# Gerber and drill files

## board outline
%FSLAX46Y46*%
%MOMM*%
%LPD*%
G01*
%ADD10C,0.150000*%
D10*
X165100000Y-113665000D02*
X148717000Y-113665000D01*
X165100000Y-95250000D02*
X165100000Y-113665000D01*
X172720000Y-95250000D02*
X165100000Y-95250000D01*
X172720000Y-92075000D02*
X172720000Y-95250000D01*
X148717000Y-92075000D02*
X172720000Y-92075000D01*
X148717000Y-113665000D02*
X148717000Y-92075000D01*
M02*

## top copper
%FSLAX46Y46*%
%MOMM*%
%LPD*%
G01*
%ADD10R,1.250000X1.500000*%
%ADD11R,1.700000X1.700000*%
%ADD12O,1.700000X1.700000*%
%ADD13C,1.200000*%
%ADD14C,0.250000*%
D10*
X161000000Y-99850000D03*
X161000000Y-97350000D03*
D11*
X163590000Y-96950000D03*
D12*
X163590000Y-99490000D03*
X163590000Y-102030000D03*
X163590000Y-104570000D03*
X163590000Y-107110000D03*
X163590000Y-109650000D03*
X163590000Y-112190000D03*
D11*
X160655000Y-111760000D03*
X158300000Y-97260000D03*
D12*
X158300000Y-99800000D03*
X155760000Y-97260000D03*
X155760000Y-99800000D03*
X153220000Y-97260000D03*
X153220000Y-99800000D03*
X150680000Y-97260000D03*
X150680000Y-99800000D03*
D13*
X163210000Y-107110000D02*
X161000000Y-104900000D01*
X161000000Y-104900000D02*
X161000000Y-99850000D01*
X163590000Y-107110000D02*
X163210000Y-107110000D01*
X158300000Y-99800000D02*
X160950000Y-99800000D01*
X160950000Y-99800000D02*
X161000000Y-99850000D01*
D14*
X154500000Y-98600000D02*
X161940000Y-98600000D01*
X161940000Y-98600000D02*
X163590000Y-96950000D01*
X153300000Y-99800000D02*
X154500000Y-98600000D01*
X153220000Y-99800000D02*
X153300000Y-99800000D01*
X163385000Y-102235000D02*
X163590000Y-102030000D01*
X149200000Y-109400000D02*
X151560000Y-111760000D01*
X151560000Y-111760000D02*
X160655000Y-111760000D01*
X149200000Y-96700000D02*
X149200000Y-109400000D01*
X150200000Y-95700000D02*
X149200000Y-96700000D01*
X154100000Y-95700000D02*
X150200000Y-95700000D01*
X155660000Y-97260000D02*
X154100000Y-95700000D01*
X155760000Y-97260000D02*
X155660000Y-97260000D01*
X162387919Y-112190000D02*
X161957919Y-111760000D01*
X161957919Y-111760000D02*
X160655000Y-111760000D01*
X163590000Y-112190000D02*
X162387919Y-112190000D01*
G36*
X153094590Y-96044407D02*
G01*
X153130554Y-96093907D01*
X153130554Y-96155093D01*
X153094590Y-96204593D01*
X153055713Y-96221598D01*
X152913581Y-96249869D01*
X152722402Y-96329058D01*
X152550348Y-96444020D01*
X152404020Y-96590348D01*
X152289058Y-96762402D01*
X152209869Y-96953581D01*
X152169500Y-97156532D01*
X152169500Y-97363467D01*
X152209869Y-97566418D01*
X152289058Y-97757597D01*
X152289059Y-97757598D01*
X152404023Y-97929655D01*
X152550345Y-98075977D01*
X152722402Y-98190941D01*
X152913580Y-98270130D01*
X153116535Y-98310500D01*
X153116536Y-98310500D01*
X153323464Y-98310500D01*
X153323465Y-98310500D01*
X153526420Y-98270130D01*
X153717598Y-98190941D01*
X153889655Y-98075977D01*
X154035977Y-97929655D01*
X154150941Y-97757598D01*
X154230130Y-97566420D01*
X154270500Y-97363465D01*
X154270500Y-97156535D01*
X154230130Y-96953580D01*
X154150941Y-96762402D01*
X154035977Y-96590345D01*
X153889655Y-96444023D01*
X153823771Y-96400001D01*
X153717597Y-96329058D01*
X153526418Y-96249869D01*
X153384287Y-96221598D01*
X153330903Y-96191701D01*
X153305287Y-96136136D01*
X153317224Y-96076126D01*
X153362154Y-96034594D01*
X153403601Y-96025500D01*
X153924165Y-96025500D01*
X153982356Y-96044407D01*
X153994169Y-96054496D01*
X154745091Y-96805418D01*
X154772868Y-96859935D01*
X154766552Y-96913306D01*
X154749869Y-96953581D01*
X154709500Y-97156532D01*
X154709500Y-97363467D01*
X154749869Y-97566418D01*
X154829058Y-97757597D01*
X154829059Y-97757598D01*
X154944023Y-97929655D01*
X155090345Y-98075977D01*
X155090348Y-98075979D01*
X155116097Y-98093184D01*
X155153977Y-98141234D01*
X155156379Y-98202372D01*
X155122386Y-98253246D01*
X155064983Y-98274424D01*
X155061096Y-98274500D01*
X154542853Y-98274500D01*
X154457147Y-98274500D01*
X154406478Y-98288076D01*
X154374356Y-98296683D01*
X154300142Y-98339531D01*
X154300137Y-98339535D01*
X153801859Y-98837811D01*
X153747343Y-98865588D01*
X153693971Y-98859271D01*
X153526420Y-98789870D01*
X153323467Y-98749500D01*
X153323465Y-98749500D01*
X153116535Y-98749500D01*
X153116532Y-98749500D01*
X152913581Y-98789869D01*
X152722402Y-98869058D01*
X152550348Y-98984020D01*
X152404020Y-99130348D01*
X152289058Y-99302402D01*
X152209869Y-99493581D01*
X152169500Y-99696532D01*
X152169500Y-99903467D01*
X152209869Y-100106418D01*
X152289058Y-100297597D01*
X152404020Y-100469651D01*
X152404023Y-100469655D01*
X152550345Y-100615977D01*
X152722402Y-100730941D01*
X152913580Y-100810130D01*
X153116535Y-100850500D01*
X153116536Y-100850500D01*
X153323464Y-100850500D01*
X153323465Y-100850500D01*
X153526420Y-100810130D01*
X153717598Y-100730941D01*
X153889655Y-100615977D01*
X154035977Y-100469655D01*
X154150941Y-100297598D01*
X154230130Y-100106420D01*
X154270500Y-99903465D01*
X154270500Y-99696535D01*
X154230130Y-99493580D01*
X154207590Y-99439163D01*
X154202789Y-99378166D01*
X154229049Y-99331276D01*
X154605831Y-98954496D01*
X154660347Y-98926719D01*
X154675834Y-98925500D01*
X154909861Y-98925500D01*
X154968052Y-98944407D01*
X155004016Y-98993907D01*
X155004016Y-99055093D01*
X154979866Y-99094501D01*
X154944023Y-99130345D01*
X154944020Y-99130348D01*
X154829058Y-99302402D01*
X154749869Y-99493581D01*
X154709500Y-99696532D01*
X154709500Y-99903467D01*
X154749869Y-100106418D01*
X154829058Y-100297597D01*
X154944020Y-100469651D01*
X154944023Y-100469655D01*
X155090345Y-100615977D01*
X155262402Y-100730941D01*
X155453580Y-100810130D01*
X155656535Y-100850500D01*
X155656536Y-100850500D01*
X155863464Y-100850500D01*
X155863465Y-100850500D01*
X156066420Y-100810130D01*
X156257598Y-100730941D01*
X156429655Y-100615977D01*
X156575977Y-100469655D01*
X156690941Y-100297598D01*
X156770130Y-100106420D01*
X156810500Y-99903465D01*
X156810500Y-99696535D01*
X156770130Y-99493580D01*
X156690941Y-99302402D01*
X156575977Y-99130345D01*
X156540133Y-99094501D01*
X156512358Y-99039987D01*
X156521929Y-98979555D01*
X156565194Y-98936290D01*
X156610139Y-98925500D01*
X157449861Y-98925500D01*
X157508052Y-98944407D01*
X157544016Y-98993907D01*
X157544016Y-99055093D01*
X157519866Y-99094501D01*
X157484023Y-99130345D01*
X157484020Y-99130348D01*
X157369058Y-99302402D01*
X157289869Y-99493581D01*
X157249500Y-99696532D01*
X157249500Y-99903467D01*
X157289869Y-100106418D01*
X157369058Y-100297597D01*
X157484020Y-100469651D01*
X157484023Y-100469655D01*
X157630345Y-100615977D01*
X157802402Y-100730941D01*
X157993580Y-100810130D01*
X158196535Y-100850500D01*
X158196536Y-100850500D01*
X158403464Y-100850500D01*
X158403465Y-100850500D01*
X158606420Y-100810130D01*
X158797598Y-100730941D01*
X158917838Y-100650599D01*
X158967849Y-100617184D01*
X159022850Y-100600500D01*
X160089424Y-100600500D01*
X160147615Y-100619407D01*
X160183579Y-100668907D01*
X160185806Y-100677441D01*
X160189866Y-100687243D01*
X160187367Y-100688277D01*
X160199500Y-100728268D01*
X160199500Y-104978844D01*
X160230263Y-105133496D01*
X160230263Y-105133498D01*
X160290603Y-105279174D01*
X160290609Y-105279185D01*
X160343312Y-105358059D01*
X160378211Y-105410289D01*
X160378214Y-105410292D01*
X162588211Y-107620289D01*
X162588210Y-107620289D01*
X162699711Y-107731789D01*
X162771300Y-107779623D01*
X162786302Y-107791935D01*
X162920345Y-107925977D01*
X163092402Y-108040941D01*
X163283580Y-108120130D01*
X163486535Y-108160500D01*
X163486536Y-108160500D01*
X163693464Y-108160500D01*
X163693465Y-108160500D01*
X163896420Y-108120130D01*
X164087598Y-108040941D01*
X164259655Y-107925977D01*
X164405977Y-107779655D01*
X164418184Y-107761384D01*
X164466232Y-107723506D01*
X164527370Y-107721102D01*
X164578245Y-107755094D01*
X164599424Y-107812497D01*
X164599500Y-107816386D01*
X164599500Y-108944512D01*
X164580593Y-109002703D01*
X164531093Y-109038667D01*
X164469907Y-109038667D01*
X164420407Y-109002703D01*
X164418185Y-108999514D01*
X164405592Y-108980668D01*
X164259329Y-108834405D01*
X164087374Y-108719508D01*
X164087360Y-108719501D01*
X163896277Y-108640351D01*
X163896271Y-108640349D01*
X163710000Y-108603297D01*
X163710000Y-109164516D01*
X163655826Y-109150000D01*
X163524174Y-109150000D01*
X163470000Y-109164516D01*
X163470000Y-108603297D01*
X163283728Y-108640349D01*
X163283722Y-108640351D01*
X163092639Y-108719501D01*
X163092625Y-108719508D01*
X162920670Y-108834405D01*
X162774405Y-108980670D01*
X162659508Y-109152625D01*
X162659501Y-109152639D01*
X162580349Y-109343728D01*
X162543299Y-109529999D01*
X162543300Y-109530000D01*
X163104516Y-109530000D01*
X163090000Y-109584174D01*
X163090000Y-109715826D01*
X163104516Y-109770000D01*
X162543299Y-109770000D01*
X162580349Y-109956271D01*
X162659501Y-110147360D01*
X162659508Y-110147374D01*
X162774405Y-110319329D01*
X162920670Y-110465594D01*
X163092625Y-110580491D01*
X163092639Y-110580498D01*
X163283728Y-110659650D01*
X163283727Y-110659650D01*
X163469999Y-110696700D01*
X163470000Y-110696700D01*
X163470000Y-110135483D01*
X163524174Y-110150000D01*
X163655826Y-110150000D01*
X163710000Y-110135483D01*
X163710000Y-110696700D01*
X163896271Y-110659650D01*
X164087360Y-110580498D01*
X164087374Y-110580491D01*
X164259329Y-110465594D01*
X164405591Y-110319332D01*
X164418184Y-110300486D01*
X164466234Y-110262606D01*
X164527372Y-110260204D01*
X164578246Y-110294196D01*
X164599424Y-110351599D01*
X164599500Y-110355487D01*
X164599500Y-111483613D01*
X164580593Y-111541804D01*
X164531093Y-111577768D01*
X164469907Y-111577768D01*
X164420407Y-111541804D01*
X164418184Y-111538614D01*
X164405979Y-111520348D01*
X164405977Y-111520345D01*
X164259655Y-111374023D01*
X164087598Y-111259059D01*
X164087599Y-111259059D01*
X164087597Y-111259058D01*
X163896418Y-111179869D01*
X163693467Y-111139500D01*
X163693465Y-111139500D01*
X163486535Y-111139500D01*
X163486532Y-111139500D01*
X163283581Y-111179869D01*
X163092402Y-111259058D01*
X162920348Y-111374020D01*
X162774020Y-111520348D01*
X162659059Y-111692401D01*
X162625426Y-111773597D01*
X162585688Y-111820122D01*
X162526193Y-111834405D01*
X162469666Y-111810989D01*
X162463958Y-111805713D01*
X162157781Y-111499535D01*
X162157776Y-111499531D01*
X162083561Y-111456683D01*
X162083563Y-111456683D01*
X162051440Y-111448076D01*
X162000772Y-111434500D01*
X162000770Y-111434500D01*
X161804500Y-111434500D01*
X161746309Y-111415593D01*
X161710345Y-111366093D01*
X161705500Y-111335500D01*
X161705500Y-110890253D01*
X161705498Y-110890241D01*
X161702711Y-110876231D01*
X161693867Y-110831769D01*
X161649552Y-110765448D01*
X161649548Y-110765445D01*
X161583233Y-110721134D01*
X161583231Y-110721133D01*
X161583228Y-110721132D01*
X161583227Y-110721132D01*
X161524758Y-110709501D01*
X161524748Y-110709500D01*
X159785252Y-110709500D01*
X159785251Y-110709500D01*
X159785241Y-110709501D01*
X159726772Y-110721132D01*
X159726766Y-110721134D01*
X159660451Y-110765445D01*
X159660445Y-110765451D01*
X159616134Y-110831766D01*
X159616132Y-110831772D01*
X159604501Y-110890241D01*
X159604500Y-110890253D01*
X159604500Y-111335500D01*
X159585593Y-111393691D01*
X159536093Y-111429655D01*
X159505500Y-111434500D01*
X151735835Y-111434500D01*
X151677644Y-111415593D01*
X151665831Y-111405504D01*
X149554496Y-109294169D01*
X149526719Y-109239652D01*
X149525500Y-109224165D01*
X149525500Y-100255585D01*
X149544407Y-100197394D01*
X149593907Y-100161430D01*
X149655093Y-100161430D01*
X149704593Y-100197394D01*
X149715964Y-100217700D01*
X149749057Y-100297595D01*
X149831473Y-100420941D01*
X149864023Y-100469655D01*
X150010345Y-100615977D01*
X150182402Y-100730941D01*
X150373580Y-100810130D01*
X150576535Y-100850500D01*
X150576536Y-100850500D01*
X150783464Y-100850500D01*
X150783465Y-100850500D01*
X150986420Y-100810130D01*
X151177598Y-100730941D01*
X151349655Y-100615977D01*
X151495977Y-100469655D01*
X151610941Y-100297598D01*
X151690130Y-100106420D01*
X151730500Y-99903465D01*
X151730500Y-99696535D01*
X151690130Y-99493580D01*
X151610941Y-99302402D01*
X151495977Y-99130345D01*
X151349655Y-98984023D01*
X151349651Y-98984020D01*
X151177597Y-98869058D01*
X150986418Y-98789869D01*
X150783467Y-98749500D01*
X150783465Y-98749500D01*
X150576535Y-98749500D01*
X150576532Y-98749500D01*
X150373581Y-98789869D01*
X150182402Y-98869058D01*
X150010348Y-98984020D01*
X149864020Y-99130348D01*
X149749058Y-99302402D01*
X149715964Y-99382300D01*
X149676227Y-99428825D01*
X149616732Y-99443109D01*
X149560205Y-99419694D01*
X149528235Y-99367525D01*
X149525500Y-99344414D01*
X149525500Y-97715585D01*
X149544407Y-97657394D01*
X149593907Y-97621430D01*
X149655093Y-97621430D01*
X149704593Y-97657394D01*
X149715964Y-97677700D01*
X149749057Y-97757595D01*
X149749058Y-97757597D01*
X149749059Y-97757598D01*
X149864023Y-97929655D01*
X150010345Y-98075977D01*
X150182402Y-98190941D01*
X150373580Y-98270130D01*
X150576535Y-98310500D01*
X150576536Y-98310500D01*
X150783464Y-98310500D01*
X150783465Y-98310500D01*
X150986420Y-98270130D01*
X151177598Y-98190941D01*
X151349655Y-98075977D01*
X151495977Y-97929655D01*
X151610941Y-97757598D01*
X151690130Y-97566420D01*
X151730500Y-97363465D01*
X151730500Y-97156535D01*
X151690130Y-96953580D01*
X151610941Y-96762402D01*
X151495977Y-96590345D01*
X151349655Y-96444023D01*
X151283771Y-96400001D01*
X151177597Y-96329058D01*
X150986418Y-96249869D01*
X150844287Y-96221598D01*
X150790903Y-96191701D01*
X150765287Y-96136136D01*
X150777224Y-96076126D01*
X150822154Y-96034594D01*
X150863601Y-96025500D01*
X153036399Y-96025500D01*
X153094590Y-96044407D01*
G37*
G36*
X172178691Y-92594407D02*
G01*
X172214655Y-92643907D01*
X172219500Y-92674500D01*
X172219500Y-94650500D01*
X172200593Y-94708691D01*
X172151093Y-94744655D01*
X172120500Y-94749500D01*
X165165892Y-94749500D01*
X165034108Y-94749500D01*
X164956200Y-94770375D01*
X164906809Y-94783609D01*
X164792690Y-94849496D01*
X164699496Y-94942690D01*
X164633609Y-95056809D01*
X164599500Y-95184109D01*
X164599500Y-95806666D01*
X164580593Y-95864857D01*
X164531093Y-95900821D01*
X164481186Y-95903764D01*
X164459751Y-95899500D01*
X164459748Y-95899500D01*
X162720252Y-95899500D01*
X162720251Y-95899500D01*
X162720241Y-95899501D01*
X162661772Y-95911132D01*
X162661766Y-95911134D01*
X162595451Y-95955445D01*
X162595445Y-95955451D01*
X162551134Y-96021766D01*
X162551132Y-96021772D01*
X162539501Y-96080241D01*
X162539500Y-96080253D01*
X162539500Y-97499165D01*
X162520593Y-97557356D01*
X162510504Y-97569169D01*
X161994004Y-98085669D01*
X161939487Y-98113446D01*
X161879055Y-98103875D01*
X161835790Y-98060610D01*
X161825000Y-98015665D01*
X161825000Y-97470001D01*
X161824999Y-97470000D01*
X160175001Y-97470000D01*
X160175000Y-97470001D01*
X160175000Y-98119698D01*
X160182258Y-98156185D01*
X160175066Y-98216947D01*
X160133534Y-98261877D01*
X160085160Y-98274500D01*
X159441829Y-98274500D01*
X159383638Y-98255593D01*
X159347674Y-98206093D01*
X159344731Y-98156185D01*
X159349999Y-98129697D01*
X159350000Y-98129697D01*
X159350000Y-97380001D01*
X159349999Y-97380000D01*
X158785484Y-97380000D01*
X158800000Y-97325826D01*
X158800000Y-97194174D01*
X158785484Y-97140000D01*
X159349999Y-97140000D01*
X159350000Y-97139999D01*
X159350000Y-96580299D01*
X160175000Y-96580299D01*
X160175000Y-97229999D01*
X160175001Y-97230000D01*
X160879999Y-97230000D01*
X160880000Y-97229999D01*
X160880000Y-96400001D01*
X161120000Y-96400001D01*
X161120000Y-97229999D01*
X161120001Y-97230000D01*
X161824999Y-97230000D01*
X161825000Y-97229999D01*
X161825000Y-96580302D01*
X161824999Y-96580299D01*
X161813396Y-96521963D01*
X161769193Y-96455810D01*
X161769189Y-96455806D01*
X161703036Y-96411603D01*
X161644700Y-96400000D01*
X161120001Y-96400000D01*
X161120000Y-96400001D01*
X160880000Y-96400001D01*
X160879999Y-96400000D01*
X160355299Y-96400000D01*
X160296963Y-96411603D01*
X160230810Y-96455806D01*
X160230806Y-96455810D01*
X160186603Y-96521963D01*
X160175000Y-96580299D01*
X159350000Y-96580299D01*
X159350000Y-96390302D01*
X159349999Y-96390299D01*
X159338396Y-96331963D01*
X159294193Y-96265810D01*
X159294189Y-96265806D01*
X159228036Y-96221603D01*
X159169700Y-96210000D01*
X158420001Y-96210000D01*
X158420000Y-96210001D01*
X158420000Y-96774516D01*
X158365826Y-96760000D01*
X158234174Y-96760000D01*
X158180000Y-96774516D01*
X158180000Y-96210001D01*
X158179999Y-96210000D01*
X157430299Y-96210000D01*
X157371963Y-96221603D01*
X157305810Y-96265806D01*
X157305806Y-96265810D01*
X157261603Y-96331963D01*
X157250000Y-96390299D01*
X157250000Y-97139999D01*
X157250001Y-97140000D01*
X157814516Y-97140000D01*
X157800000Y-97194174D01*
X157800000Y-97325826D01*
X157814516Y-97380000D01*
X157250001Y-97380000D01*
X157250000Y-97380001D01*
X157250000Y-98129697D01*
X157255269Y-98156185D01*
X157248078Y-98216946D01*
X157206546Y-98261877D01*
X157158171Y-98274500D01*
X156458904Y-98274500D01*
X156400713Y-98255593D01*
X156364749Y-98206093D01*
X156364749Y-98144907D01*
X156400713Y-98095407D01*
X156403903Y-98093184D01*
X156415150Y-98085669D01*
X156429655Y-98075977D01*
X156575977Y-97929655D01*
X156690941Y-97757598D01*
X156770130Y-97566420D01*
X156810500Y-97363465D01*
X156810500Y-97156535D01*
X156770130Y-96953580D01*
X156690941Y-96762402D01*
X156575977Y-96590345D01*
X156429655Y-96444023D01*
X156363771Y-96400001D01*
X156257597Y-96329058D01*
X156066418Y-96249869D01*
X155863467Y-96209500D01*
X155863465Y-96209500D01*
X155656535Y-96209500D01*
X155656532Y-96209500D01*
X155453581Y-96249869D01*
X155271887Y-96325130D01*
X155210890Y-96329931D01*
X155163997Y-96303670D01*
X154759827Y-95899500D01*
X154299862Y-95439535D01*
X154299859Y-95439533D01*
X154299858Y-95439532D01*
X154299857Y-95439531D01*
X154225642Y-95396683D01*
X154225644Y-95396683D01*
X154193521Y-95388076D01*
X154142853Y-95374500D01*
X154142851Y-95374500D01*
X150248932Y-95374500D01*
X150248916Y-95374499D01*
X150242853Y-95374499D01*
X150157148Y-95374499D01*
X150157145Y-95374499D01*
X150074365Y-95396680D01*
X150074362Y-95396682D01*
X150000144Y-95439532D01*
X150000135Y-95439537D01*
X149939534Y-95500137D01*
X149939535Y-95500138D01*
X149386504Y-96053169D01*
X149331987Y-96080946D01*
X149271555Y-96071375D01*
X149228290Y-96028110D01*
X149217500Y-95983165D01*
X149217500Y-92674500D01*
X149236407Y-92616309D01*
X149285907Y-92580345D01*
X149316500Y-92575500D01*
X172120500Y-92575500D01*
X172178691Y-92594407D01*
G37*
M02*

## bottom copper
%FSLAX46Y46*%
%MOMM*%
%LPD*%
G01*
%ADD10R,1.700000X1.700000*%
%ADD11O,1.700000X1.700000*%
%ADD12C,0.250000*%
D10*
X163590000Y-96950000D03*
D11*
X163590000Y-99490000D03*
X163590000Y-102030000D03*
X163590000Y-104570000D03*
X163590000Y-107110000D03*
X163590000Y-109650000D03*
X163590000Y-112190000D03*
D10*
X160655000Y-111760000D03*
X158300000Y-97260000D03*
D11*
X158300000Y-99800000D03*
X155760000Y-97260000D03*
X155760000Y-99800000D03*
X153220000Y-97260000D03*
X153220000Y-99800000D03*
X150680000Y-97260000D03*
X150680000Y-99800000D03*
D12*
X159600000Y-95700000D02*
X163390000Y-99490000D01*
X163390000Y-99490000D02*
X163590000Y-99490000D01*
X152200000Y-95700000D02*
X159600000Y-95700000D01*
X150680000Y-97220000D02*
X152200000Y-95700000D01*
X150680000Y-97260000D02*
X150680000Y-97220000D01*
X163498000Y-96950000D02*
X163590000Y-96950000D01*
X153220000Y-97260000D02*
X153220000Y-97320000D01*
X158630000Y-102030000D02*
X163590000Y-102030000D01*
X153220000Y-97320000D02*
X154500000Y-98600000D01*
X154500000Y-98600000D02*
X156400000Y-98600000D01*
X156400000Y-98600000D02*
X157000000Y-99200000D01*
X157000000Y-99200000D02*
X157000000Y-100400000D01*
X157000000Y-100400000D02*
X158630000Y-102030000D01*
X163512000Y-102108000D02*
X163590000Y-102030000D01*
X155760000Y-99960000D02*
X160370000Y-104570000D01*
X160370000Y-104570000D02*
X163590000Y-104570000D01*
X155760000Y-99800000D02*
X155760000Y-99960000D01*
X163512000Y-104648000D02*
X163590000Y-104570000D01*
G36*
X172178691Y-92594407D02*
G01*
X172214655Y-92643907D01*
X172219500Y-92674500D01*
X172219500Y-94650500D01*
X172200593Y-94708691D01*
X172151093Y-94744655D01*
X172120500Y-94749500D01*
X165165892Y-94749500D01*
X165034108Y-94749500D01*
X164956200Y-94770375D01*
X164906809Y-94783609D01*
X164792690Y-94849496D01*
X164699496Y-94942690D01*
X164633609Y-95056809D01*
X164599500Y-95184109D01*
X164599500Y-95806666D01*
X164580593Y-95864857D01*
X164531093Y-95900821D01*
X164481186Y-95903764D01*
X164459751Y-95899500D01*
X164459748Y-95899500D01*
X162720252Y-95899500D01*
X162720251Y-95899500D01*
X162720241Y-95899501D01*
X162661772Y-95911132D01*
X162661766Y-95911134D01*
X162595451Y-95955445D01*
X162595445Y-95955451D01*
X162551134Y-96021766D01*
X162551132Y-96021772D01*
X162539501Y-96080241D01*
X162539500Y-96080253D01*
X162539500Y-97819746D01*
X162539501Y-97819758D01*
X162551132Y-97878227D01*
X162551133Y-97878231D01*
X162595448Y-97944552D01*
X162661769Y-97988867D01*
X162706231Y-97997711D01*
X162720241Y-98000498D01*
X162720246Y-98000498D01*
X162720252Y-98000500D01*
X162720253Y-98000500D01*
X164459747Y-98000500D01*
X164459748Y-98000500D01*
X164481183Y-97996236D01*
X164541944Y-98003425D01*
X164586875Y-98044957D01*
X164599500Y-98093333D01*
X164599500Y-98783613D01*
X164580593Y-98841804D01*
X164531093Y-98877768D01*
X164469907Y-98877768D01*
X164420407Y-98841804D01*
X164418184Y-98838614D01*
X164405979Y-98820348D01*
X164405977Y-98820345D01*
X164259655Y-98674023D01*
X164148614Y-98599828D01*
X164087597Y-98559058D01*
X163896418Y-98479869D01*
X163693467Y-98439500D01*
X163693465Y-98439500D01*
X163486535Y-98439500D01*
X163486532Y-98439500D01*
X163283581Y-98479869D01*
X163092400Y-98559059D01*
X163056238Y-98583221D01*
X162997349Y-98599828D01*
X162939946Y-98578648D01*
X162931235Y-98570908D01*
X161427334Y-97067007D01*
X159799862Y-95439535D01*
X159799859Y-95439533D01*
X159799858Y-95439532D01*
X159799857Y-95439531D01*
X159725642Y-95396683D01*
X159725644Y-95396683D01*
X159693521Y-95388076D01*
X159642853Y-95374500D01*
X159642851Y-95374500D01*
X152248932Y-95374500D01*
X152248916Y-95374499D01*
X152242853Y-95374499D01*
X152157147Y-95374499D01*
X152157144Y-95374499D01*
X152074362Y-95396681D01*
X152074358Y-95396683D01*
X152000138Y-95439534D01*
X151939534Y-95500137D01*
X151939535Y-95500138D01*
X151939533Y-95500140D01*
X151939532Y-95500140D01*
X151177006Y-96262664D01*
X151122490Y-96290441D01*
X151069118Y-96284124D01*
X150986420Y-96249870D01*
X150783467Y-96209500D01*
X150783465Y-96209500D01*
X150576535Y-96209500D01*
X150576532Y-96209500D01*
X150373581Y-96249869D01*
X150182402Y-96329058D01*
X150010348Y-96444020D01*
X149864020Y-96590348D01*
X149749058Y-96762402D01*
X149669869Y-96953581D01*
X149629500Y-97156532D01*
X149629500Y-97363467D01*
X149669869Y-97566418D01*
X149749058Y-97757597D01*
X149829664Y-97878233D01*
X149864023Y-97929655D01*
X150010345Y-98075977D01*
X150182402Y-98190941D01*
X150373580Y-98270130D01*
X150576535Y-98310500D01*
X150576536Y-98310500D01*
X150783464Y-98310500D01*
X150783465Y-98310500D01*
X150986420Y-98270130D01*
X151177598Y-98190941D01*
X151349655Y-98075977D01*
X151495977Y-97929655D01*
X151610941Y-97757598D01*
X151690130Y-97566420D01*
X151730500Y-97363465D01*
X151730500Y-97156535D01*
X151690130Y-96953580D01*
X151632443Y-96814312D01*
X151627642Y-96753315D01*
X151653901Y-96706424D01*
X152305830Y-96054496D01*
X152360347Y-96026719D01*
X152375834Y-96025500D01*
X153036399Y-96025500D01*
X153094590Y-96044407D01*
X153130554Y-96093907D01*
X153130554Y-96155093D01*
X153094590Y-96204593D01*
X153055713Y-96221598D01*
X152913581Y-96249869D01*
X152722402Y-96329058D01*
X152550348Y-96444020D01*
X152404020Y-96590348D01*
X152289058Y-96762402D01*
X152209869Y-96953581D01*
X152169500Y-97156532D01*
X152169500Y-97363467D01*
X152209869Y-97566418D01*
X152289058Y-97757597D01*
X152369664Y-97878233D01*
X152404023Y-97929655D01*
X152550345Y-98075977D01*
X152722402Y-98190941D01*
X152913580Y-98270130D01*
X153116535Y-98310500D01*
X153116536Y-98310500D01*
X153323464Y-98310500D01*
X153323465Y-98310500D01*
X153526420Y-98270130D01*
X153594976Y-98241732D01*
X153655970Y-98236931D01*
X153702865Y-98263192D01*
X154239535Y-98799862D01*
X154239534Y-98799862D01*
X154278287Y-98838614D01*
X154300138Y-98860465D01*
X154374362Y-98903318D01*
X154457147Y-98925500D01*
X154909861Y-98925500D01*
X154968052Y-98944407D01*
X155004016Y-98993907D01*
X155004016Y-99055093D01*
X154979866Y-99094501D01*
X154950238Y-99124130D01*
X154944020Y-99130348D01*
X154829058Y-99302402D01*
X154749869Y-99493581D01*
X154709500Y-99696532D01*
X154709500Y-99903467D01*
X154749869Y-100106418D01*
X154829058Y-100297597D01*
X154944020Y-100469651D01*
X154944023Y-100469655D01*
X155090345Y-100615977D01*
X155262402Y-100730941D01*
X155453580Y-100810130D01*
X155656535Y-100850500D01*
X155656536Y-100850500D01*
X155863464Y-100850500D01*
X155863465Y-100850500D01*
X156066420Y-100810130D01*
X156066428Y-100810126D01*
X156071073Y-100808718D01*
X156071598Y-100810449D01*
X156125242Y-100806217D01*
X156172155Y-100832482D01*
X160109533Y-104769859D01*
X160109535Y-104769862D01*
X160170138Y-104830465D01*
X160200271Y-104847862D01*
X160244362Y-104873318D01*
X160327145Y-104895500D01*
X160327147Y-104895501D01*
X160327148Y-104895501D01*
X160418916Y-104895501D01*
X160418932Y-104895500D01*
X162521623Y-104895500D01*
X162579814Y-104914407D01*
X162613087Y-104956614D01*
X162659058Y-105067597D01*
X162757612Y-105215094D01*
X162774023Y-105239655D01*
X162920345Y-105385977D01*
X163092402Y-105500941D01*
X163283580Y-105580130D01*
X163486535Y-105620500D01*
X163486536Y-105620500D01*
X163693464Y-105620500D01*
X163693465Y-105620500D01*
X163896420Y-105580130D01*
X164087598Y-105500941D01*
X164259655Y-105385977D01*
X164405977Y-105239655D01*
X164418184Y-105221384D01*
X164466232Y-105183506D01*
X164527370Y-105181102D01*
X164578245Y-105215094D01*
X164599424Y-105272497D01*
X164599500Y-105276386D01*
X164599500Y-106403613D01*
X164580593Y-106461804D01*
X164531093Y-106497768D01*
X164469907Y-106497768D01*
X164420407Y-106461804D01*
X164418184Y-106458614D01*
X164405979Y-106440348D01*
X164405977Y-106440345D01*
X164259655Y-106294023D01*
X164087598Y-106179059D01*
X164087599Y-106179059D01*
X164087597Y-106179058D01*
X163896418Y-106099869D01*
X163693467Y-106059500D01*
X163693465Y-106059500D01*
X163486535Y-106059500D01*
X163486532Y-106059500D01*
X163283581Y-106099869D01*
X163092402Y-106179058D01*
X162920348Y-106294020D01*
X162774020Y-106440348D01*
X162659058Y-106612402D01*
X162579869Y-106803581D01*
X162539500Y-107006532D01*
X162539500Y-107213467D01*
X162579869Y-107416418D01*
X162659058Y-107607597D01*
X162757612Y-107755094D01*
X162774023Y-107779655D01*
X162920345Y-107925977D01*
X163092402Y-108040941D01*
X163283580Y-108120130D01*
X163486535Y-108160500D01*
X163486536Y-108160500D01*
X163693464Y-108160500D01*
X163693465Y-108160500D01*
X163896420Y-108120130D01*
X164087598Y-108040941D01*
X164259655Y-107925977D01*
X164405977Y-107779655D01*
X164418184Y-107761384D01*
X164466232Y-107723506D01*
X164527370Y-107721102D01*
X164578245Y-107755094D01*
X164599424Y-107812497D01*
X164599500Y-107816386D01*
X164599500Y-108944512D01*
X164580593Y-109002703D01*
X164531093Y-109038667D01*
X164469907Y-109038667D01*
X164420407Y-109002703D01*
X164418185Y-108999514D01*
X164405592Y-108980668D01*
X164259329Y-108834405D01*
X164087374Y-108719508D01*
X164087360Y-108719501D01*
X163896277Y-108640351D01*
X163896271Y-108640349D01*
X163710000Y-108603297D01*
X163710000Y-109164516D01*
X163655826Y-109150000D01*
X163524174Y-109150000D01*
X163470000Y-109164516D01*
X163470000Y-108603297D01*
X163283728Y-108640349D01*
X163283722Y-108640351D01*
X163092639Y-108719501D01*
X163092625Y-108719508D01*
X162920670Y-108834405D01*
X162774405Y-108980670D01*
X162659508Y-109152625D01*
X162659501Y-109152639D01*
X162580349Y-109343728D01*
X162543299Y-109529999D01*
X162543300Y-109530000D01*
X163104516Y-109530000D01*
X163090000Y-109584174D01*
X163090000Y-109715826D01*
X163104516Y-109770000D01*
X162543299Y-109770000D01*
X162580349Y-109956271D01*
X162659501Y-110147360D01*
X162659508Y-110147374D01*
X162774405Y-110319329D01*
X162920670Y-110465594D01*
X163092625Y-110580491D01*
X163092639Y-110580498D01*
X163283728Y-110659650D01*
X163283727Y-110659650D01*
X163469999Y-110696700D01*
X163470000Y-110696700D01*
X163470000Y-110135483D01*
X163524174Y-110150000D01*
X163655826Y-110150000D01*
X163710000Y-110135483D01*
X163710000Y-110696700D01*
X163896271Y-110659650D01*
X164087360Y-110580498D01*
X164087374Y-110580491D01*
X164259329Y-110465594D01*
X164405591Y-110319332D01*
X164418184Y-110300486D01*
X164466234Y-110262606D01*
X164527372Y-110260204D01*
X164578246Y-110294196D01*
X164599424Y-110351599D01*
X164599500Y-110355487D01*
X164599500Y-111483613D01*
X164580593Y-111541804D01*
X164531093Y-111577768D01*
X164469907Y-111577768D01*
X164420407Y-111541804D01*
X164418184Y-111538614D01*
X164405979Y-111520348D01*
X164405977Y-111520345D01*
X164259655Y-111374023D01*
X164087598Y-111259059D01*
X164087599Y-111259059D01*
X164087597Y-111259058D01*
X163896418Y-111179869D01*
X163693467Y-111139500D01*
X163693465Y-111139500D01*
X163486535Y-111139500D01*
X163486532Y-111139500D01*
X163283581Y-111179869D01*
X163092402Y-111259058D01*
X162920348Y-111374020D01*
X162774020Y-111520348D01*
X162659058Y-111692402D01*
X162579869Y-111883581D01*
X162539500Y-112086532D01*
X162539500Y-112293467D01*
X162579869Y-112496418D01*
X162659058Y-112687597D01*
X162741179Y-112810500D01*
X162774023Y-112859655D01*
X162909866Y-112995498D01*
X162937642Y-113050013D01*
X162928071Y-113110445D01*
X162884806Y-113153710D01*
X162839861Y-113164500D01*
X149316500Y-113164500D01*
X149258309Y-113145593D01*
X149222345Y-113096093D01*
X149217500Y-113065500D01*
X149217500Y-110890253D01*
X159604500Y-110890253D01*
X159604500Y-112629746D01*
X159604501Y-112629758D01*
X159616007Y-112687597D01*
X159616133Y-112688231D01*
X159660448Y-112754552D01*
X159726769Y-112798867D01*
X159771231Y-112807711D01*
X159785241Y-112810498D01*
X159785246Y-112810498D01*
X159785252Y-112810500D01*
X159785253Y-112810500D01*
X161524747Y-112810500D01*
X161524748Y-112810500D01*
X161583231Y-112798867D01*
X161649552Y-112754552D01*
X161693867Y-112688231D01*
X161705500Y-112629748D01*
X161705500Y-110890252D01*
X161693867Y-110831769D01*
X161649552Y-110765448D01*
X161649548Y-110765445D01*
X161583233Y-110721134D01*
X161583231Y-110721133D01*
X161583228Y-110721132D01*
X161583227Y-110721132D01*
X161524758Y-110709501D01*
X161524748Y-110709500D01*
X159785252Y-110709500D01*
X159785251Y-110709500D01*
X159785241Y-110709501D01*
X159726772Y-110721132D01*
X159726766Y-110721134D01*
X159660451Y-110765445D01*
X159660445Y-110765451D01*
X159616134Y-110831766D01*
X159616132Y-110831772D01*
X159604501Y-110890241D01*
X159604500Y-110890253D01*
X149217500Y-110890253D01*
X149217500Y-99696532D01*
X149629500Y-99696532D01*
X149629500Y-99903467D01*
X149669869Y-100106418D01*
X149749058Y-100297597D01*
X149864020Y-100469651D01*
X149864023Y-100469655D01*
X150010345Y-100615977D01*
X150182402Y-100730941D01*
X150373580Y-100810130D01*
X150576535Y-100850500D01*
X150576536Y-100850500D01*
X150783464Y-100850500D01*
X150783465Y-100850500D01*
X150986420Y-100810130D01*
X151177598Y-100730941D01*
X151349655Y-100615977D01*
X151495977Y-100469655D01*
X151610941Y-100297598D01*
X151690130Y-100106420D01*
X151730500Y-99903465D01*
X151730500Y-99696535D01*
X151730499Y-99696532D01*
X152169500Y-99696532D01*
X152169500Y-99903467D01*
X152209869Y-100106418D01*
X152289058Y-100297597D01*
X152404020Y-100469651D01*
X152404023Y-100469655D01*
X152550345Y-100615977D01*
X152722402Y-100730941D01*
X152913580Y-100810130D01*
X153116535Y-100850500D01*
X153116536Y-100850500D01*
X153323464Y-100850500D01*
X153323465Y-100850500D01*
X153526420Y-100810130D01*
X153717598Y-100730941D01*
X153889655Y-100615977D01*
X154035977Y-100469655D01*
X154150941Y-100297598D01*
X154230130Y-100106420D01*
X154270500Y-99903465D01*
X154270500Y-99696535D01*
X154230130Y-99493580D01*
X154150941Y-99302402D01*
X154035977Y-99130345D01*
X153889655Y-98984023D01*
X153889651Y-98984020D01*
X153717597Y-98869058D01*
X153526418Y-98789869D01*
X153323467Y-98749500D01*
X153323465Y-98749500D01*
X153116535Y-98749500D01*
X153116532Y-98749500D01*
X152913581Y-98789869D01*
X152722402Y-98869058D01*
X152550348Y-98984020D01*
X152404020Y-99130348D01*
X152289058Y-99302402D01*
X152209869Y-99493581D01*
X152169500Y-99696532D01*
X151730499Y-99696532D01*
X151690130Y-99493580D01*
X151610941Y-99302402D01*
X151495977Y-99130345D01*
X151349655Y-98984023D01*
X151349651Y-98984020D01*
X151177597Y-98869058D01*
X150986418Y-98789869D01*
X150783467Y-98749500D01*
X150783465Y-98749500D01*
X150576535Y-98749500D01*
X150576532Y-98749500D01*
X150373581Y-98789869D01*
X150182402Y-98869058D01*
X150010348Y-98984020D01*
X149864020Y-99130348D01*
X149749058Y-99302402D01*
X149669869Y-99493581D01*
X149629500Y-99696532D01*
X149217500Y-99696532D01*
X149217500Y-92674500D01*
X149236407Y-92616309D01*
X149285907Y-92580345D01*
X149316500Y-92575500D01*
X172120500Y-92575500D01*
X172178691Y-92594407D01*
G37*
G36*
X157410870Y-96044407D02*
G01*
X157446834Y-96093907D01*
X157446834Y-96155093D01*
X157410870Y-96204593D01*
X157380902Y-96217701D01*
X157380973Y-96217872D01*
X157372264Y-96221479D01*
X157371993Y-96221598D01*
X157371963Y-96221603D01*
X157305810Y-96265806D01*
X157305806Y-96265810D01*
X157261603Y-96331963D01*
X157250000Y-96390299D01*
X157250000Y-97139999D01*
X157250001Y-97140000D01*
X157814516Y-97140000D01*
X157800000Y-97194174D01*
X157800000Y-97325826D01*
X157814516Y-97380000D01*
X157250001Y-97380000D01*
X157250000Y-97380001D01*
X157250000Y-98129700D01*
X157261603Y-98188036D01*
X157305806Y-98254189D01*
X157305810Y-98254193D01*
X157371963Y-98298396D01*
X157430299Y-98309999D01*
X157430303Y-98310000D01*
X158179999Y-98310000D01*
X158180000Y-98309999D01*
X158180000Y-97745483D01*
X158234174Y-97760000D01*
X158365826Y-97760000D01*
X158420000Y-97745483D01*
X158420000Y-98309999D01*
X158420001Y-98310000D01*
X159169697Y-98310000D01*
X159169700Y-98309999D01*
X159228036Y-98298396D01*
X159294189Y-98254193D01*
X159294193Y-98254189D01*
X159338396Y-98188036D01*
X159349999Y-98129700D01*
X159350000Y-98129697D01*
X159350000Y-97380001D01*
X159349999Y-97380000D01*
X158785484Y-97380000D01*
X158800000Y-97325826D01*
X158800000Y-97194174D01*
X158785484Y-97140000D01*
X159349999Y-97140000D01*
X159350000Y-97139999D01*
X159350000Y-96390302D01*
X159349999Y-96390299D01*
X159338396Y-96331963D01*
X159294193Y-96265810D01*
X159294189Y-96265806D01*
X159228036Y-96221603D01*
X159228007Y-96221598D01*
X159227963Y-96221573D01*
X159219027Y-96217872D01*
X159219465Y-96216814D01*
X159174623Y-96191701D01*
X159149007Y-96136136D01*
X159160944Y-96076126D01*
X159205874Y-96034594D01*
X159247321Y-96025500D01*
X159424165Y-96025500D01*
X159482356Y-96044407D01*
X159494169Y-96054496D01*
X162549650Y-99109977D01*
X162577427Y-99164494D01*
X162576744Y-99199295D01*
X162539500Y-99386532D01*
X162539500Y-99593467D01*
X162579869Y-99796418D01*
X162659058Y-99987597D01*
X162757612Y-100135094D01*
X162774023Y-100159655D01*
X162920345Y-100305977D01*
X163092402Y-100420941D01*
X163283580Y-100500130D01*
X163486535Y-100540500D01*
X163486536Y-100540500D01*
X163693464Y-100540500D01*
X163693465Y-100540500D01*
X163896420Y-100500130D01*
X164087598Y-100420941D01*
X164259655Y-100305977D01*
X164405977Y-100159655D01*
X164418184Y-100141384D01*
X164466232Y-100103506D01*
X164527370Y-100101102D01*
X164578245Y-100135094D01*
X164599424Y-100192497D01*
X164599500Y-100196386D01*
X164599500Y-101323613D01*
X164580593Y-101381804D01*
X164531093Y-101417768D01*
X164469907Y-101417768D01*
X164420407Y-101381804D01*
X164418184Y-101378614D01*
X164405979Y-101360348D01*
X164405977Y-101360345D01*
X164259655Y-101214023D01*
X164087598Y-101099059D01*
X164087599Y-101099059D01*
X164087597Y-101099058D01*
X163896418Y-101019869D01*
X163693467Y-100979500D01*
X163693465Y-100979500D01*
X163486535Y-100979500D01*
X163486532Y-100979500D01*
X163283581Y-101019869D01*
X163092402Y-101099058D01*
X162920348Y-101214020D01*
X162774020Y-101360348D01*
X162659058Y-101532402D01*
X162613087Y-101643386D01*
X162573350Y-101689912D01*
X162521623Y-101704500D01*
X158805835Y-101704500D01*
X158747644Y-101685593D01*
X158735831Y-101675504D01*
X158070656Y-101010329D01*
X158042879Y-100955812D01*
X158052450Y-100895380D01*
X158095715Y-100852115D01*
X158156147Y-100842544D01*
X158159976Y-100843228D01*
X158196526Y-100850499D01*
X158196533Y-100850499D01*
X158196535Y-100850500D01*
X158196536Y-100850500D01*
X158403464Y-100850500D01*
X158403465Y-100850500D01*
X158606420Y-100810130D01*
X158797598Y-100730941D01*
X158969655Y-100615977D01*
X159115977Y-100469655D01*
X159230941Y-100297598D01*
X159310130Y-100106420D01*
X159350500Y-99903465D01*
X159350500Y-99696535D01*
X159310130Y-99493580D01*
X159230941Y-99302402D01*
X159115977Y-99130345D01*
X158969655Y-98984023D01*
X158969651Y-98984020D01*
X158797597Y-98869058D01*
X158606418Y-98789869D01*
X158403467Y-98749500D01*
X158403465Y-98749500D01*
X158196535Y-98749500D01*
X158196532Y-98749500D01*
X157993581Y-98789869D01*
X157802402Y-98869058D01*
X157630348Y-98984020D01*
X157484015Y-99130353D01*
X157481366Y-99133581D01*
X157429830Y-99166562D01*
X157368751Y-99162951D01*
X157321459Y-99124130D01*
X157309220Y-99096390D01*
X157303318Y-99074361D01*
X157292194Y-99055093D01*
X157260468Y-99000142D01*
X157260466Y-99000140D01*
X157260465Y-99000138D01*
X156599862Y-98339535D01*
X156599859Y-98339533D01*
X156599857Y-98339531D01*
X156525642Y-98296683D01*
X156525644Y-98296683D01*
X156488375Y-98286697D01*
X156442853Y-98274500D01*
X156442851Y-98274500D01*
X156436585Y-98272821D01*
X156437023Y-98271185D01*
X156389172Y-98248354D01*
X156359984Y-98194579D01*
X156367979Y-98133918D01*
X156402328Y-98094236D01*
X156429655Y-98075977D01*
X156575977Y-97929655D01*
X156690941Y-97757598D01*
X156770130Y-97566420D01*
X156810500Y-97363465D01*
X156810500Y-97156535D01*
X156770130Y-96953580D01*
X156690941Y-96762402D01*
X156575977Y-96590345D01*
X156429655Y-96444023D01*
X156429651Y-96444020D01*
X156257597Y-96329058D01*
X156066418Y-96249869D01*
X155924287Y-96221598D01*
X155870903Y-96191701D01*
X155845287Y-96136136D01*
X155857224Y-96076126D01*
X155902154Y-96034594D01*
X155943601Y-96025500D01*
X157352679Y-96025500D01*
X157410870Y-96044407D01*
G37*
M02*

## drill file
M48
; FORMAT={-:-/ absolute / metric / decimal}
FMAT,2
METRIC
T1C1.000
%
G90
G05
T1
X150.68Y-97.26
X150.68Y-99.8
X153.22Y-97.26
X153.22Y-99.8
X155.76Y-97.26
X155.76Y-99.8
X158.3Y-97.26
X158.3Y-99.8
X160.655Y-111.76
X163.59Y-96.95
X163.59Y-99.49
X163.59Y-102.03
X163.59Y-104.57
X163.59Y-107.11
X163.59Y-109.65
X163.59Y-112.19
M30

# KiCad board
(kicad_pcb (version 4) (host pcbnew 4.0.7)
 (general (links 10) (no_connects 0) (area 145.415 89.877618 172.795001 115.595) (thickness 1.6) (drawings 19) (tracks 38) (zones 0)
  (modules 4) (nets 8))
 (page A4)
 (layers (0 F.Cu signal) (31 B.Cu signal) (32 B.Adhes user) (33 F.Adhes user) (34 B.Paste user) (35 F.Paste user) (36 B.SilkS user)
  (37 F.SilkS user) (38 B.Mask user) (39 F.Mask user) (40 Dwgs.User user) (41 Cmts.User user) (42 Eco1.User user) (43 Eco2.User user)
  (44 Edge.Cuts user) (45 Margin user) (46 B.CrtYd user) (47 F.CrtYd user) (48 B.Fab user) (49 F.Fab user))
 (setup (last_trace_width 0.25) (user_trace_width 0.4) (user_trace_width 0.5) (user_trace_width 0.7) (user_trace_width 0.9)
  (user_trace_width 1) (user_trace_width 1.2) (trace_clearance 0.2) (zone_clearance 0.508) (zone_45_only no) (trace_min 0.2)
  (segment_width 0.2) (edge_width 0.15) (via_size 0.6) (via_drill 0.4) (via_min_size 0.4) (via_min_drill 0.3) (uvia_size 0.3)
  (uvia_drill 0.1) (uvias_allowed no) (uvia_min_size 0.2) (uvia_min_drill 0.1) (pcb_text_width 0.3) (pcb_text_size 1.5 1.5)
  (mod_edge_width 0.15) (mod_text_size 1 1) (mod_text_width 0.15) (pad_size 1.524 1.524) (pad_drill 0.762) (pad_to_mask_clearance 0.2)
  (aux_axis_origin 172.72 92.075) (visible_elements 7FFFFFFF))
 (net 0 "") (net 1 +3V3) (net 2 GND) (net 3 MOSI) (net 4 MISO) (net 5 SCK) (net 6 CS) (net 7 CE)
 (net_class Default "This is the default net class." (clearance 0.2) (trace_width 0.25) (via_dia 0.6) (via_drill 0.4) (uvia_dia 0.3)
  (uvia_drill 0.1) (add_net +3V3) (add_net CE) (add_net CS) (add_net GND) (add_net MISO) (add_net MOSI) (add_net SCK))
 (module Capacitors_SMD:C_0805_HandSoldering (layer F.Cu) (at 161 98.6 90)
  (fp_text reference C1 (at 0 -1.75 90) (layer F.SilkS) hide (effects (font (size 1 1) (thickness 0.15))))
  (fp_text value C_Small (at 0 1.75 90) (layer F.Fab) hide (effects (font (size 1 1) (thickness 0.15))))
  (pad 1 smd rect (at -1.25 0 90) (size 1.5 1.25) (layers F.Cu F.Paste F.Mask) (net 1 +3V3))
  (pad 2 smd rect (at 1.25 0 90) (size 1.5 1.25) (layers F.Cu F.Paste F.Mask) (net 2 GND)))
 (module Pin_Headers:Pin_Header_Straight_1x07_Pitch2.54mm (layer F.Cu) (at 163.59 96.95)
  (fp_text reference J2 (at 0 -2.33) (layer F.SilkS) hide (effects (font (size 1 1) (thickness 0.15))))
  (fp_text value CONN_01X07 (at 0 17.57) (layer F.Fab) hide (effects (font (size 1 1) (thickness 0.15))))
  (pad 1 thru_hole rect (at 0 0) (size 1.7 1.7) (drill 1) (layers *.Cu *.Mask) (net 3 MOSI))
  (pad 2 thru_hole oval (at 0 2.54) (size 1.7 1.7) (drill 1) (layers *.Cu *.Mask) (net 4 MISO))
  (pad 3 thru_hole oval (at 0 5.08) (size 1.7 1.7) (drill 1) (layers *.Cu *.Mask) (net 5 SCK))
  (pad 4 thru_hole oval (at 0 7.62) (size 1.7 1.7) (drill 1) (layers *.Cu *.Mask) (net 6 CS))
  (pad 5 thru_hole oval (at 0 10.16) (size 1.7 1.7) (drill 1) (layers *.Cu *.Mask) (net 1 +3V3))
  (pad 6 thru_hole oval (at 0 12.7) (size 1.7 1.7) (drill 1) (layers *.Cu *.Mask) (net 2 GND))
  (pad 7 thru_hole oval (at 0 15.24) (size 1.7 1.7) (drill 1) (layers *.Cu *.Mask) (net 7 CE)))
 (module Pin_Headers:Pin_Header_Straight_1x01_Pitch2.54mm (layer F.Cu) (at 160.655 111.76)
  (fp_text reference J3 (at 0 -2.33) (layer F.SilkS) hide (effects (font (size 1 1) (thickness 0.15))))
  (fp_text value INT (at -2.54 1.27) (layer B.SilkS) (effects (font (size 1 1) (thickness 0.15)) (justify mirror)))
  (pad 1 thru_hole rect (at 0 0) (size 1.7 1.7) (drill 1) (layers *.Cu *.Mask) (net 7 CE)))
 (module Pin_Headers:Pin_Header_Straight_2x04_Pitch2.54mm (layer F.Cu) (at 158.3 97.26 270)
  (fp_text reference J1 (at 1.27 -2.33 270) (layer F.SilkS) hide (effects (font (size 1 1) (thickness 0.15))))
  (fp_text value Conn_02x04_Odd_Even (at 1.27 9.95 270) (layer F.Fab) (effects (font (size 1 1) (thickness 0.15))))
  (pad 1 thru_hole rect (at 0 0 270) (size 1.7 1.7) (drill 1) (layers *.Cu *.Mask) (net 2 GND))
  (pad 2 thru_hole oval (at 2.54 0 270) (size 1.7 1.7) (drill 1) (layers *.Cu *.Mask) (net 1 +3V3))
  (pad 3 thru_hole oval (at 0 2.54 270) (size 1.7 1.7) (drill 1) (layers *.Cu *.Mask) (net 7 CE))
  (pad 4 thru_hole oval (at 2.54 2.54 270) (size 1.7 1.7) (drill 1) (layers *.Cu *.Mask) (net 6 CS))
  (pad 5 thru_hole oval (at 0 5.08 270) (size 1.7 1.7) (drill 1) (layers *.Cu *.Mask) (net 5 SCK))
  (pad 6 thru_hole oval (at 2.54 5.08 270) (size 1.7 1.7) (drill 1) (layers *.Cu *.Mask) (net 3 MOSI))
  (pad 7 thru_hole oval (at 0 7.62 270) (size 1.7 1.7) (drill 1) (layers *.Cu *.Mask) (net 4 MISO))
  (pad 8 thru_hole oval (at 2.54 7.62 270) (size 1.7 1.7) (drill 1) (layers *.Cu *.Mask)))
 (gr_line (start 165.1 113.665) (end 148.717 113.665) (layer Edge.Cuts) (width 0.15))
 (gr_line (start 165.1 95.25) (end 165.1 113.665) (layer Edge.Cuts) (width 0.15))
 (gr_line (start 172.72 95.25) (end 165.1 95.25) (layer Edge.Cuts) (width 0.15))
 (gr_line (start 172.72 92.075) (end 172.72 95.25) (layer Edge.Cuts) (width 0.15))
 (gr_line (start 148.717 92.075) (end 172.72 92.075) (layer Edge.Cuts) (width 0.15))
 (gr_line (start 148.717 113.665) (end 148.717 92.075) (layer Edge.Cuts) (width 0.15))
 (segment (start 163.21 107.11) (end 161 104.9) (width 1.2) (layer F.Cu) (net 1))
 (segment (start 161 104.9) (end 161 99.85) (width 1.2) (layer F.Cu) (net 1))
 (segment (start 163.59 107.11) (end 163.21 107.11) (width 1.2) (layer F.Cu) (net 1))
 (segment (start 158.3 99.8) (end 160.95 99.8) (width 1.2) (layer F.Cu) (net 1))
 (segment (start 160.95 99.8) (end 161 99.85) (width 1.2) (layer F.Cu) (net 1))
 (segment (start 159.6 95.7) (end 163.39 99.49) (width 0.25) (layer B.Cu) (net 4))
 (segment (start 163.39 99.49) (end 163.59 99.49) (width 0.25) (layer B.Cu) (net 4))
 (segment (start 152.2 95.7) (end 159.6 95.7) (width 0.25) (layer B.Cu) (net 4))
 (segment (start 150.68 97.22) (end 152.2 95.7) (width 0.25) (layer B.Cu) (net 4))
 (segment (start 150.68 97.26) (end 150.68 97.22) (width 0.25) (layer B.Cu) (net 4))
 (segment (start 154.5 98.6) (end 161.94 98.6) (width 0.25) (layer F.Cu) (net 3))
 (segment (start 161.94 98.6) (end 163.59 96.95) (width 0.25) (layer F.Cu) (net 3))
 (segment (start 153.3 99.8) (end 154.5 98.6) (width 0.25) (layer F.Cu) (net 3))
 (segment (start 153.22 99.8) (end 153.3 99.8) (width 0.25) (layer F.Cu) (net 3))
 (segment (start 163.498 96.95) (end 163.59 96.95) (width 0.25) (layer B.Cu) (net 3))
 (segment (start 153.22 97.26) (end 153.22 97.32) (width 0.25) (layer B.Cu) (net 5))
 (segment (start 158.63 102.03) (end 163.59 102.03) (width 0.25) (layer B.Cu) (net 5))
 (segment (start 153.22 97.32) (end 154.5 98.6) (width 0.25) (layer B.Cu) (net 5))
 (segment (start 154.5 98.6) (end 156.4 98.6) (width 0.25) (layer B.Cu) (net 5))
 (segment (start 156.4 98.6) (end 157 99.2) (width 0.25) (layer B.Cu) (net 5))
 (segment (start 157 99.2) (end 157 100.4) (width 0.25) (layer B.Cu) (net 5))
 (segment (start 157 100.4) (end 158.63 102.03) (width 0.25) (layer B.Cu) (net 5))
 (segment (start 163.512 102.108) (end 163.59 102.03) (width 0.25) (layer B.Cu) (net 5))
 (segment (start 163.385 102.235) (end 163.59 102.03) (width 0.25) (layer F.Cu) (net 5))
 (segment (start 155.76 99.96) (end 160.37 104.57) (width 0.25) (layer B.Cu) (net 6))
 (segment (start 160.37 104.57) (end 163.59 104.57) (width 0.25) (layer B.Cu) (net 6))
 (segment (start 155.76 99.8) (end 155.76 99.96) (width 0.25) (layer B.Cu) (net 6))
 (segment (start 163.512 104.648) (end 163.59 104.57) (width 0.25) (layer B.Cu) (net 6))
 (segment (start 149.2 109.4) (end 151.56 111.76) (width 0.25) (layer F.Cu) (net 7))
 (segment (start 151.56 111.76) (end 160.655 111.76) (width 0.25) (layer F.Cu) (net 7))
 (segment (start 149.2 96.7) (end 149.2 109.4) (width 0.25) (layer F.Cu) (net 7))
 (segment (start 150.2 95.7) (end 149.2 96.7) (width 0.25) (layer F.Cu) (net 7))
 (segment (start 154.1 95.7) (end 150.2 95.7) (width 0.25) (layer F.Cu) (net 7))
 (segment (start 155.66 97.26) (end 154.1 95.7) (width 0.25) (layer F.Cu) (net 7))
 (segment (start 155.76 97.26) (end 155.66 97.26) (width 0.25) (layer F.Cu) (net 7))
 (segment (start 162.387919 112.19) (end 161.957919 111.76) (width 0.25) (layer F.Cu) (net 7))
 (segment (start 161.957919 111.76) (end 160.655 111.76) (width 0.25) (layer F.Cu) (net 7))
 (segment (start 163.59 112.19) (end 162.387919 112.19) (width 0.25) (layer F.Cu) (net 7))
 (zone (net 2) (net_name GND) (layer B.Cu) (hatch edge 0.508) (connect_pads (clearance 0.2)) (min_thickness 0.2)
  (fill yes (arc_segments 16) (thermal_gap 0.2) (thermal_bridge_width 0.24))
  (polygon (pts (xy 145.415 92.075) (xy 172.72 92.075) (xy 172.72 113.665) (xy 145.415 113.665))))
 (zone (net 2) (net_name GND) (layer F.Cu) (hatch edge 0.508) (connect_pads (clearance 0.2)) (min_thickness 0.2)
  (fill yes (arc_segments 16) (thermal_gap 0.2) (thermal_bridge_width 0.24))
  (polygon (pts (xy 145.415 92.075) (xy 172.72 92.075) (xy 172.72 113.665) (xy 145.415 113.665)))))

